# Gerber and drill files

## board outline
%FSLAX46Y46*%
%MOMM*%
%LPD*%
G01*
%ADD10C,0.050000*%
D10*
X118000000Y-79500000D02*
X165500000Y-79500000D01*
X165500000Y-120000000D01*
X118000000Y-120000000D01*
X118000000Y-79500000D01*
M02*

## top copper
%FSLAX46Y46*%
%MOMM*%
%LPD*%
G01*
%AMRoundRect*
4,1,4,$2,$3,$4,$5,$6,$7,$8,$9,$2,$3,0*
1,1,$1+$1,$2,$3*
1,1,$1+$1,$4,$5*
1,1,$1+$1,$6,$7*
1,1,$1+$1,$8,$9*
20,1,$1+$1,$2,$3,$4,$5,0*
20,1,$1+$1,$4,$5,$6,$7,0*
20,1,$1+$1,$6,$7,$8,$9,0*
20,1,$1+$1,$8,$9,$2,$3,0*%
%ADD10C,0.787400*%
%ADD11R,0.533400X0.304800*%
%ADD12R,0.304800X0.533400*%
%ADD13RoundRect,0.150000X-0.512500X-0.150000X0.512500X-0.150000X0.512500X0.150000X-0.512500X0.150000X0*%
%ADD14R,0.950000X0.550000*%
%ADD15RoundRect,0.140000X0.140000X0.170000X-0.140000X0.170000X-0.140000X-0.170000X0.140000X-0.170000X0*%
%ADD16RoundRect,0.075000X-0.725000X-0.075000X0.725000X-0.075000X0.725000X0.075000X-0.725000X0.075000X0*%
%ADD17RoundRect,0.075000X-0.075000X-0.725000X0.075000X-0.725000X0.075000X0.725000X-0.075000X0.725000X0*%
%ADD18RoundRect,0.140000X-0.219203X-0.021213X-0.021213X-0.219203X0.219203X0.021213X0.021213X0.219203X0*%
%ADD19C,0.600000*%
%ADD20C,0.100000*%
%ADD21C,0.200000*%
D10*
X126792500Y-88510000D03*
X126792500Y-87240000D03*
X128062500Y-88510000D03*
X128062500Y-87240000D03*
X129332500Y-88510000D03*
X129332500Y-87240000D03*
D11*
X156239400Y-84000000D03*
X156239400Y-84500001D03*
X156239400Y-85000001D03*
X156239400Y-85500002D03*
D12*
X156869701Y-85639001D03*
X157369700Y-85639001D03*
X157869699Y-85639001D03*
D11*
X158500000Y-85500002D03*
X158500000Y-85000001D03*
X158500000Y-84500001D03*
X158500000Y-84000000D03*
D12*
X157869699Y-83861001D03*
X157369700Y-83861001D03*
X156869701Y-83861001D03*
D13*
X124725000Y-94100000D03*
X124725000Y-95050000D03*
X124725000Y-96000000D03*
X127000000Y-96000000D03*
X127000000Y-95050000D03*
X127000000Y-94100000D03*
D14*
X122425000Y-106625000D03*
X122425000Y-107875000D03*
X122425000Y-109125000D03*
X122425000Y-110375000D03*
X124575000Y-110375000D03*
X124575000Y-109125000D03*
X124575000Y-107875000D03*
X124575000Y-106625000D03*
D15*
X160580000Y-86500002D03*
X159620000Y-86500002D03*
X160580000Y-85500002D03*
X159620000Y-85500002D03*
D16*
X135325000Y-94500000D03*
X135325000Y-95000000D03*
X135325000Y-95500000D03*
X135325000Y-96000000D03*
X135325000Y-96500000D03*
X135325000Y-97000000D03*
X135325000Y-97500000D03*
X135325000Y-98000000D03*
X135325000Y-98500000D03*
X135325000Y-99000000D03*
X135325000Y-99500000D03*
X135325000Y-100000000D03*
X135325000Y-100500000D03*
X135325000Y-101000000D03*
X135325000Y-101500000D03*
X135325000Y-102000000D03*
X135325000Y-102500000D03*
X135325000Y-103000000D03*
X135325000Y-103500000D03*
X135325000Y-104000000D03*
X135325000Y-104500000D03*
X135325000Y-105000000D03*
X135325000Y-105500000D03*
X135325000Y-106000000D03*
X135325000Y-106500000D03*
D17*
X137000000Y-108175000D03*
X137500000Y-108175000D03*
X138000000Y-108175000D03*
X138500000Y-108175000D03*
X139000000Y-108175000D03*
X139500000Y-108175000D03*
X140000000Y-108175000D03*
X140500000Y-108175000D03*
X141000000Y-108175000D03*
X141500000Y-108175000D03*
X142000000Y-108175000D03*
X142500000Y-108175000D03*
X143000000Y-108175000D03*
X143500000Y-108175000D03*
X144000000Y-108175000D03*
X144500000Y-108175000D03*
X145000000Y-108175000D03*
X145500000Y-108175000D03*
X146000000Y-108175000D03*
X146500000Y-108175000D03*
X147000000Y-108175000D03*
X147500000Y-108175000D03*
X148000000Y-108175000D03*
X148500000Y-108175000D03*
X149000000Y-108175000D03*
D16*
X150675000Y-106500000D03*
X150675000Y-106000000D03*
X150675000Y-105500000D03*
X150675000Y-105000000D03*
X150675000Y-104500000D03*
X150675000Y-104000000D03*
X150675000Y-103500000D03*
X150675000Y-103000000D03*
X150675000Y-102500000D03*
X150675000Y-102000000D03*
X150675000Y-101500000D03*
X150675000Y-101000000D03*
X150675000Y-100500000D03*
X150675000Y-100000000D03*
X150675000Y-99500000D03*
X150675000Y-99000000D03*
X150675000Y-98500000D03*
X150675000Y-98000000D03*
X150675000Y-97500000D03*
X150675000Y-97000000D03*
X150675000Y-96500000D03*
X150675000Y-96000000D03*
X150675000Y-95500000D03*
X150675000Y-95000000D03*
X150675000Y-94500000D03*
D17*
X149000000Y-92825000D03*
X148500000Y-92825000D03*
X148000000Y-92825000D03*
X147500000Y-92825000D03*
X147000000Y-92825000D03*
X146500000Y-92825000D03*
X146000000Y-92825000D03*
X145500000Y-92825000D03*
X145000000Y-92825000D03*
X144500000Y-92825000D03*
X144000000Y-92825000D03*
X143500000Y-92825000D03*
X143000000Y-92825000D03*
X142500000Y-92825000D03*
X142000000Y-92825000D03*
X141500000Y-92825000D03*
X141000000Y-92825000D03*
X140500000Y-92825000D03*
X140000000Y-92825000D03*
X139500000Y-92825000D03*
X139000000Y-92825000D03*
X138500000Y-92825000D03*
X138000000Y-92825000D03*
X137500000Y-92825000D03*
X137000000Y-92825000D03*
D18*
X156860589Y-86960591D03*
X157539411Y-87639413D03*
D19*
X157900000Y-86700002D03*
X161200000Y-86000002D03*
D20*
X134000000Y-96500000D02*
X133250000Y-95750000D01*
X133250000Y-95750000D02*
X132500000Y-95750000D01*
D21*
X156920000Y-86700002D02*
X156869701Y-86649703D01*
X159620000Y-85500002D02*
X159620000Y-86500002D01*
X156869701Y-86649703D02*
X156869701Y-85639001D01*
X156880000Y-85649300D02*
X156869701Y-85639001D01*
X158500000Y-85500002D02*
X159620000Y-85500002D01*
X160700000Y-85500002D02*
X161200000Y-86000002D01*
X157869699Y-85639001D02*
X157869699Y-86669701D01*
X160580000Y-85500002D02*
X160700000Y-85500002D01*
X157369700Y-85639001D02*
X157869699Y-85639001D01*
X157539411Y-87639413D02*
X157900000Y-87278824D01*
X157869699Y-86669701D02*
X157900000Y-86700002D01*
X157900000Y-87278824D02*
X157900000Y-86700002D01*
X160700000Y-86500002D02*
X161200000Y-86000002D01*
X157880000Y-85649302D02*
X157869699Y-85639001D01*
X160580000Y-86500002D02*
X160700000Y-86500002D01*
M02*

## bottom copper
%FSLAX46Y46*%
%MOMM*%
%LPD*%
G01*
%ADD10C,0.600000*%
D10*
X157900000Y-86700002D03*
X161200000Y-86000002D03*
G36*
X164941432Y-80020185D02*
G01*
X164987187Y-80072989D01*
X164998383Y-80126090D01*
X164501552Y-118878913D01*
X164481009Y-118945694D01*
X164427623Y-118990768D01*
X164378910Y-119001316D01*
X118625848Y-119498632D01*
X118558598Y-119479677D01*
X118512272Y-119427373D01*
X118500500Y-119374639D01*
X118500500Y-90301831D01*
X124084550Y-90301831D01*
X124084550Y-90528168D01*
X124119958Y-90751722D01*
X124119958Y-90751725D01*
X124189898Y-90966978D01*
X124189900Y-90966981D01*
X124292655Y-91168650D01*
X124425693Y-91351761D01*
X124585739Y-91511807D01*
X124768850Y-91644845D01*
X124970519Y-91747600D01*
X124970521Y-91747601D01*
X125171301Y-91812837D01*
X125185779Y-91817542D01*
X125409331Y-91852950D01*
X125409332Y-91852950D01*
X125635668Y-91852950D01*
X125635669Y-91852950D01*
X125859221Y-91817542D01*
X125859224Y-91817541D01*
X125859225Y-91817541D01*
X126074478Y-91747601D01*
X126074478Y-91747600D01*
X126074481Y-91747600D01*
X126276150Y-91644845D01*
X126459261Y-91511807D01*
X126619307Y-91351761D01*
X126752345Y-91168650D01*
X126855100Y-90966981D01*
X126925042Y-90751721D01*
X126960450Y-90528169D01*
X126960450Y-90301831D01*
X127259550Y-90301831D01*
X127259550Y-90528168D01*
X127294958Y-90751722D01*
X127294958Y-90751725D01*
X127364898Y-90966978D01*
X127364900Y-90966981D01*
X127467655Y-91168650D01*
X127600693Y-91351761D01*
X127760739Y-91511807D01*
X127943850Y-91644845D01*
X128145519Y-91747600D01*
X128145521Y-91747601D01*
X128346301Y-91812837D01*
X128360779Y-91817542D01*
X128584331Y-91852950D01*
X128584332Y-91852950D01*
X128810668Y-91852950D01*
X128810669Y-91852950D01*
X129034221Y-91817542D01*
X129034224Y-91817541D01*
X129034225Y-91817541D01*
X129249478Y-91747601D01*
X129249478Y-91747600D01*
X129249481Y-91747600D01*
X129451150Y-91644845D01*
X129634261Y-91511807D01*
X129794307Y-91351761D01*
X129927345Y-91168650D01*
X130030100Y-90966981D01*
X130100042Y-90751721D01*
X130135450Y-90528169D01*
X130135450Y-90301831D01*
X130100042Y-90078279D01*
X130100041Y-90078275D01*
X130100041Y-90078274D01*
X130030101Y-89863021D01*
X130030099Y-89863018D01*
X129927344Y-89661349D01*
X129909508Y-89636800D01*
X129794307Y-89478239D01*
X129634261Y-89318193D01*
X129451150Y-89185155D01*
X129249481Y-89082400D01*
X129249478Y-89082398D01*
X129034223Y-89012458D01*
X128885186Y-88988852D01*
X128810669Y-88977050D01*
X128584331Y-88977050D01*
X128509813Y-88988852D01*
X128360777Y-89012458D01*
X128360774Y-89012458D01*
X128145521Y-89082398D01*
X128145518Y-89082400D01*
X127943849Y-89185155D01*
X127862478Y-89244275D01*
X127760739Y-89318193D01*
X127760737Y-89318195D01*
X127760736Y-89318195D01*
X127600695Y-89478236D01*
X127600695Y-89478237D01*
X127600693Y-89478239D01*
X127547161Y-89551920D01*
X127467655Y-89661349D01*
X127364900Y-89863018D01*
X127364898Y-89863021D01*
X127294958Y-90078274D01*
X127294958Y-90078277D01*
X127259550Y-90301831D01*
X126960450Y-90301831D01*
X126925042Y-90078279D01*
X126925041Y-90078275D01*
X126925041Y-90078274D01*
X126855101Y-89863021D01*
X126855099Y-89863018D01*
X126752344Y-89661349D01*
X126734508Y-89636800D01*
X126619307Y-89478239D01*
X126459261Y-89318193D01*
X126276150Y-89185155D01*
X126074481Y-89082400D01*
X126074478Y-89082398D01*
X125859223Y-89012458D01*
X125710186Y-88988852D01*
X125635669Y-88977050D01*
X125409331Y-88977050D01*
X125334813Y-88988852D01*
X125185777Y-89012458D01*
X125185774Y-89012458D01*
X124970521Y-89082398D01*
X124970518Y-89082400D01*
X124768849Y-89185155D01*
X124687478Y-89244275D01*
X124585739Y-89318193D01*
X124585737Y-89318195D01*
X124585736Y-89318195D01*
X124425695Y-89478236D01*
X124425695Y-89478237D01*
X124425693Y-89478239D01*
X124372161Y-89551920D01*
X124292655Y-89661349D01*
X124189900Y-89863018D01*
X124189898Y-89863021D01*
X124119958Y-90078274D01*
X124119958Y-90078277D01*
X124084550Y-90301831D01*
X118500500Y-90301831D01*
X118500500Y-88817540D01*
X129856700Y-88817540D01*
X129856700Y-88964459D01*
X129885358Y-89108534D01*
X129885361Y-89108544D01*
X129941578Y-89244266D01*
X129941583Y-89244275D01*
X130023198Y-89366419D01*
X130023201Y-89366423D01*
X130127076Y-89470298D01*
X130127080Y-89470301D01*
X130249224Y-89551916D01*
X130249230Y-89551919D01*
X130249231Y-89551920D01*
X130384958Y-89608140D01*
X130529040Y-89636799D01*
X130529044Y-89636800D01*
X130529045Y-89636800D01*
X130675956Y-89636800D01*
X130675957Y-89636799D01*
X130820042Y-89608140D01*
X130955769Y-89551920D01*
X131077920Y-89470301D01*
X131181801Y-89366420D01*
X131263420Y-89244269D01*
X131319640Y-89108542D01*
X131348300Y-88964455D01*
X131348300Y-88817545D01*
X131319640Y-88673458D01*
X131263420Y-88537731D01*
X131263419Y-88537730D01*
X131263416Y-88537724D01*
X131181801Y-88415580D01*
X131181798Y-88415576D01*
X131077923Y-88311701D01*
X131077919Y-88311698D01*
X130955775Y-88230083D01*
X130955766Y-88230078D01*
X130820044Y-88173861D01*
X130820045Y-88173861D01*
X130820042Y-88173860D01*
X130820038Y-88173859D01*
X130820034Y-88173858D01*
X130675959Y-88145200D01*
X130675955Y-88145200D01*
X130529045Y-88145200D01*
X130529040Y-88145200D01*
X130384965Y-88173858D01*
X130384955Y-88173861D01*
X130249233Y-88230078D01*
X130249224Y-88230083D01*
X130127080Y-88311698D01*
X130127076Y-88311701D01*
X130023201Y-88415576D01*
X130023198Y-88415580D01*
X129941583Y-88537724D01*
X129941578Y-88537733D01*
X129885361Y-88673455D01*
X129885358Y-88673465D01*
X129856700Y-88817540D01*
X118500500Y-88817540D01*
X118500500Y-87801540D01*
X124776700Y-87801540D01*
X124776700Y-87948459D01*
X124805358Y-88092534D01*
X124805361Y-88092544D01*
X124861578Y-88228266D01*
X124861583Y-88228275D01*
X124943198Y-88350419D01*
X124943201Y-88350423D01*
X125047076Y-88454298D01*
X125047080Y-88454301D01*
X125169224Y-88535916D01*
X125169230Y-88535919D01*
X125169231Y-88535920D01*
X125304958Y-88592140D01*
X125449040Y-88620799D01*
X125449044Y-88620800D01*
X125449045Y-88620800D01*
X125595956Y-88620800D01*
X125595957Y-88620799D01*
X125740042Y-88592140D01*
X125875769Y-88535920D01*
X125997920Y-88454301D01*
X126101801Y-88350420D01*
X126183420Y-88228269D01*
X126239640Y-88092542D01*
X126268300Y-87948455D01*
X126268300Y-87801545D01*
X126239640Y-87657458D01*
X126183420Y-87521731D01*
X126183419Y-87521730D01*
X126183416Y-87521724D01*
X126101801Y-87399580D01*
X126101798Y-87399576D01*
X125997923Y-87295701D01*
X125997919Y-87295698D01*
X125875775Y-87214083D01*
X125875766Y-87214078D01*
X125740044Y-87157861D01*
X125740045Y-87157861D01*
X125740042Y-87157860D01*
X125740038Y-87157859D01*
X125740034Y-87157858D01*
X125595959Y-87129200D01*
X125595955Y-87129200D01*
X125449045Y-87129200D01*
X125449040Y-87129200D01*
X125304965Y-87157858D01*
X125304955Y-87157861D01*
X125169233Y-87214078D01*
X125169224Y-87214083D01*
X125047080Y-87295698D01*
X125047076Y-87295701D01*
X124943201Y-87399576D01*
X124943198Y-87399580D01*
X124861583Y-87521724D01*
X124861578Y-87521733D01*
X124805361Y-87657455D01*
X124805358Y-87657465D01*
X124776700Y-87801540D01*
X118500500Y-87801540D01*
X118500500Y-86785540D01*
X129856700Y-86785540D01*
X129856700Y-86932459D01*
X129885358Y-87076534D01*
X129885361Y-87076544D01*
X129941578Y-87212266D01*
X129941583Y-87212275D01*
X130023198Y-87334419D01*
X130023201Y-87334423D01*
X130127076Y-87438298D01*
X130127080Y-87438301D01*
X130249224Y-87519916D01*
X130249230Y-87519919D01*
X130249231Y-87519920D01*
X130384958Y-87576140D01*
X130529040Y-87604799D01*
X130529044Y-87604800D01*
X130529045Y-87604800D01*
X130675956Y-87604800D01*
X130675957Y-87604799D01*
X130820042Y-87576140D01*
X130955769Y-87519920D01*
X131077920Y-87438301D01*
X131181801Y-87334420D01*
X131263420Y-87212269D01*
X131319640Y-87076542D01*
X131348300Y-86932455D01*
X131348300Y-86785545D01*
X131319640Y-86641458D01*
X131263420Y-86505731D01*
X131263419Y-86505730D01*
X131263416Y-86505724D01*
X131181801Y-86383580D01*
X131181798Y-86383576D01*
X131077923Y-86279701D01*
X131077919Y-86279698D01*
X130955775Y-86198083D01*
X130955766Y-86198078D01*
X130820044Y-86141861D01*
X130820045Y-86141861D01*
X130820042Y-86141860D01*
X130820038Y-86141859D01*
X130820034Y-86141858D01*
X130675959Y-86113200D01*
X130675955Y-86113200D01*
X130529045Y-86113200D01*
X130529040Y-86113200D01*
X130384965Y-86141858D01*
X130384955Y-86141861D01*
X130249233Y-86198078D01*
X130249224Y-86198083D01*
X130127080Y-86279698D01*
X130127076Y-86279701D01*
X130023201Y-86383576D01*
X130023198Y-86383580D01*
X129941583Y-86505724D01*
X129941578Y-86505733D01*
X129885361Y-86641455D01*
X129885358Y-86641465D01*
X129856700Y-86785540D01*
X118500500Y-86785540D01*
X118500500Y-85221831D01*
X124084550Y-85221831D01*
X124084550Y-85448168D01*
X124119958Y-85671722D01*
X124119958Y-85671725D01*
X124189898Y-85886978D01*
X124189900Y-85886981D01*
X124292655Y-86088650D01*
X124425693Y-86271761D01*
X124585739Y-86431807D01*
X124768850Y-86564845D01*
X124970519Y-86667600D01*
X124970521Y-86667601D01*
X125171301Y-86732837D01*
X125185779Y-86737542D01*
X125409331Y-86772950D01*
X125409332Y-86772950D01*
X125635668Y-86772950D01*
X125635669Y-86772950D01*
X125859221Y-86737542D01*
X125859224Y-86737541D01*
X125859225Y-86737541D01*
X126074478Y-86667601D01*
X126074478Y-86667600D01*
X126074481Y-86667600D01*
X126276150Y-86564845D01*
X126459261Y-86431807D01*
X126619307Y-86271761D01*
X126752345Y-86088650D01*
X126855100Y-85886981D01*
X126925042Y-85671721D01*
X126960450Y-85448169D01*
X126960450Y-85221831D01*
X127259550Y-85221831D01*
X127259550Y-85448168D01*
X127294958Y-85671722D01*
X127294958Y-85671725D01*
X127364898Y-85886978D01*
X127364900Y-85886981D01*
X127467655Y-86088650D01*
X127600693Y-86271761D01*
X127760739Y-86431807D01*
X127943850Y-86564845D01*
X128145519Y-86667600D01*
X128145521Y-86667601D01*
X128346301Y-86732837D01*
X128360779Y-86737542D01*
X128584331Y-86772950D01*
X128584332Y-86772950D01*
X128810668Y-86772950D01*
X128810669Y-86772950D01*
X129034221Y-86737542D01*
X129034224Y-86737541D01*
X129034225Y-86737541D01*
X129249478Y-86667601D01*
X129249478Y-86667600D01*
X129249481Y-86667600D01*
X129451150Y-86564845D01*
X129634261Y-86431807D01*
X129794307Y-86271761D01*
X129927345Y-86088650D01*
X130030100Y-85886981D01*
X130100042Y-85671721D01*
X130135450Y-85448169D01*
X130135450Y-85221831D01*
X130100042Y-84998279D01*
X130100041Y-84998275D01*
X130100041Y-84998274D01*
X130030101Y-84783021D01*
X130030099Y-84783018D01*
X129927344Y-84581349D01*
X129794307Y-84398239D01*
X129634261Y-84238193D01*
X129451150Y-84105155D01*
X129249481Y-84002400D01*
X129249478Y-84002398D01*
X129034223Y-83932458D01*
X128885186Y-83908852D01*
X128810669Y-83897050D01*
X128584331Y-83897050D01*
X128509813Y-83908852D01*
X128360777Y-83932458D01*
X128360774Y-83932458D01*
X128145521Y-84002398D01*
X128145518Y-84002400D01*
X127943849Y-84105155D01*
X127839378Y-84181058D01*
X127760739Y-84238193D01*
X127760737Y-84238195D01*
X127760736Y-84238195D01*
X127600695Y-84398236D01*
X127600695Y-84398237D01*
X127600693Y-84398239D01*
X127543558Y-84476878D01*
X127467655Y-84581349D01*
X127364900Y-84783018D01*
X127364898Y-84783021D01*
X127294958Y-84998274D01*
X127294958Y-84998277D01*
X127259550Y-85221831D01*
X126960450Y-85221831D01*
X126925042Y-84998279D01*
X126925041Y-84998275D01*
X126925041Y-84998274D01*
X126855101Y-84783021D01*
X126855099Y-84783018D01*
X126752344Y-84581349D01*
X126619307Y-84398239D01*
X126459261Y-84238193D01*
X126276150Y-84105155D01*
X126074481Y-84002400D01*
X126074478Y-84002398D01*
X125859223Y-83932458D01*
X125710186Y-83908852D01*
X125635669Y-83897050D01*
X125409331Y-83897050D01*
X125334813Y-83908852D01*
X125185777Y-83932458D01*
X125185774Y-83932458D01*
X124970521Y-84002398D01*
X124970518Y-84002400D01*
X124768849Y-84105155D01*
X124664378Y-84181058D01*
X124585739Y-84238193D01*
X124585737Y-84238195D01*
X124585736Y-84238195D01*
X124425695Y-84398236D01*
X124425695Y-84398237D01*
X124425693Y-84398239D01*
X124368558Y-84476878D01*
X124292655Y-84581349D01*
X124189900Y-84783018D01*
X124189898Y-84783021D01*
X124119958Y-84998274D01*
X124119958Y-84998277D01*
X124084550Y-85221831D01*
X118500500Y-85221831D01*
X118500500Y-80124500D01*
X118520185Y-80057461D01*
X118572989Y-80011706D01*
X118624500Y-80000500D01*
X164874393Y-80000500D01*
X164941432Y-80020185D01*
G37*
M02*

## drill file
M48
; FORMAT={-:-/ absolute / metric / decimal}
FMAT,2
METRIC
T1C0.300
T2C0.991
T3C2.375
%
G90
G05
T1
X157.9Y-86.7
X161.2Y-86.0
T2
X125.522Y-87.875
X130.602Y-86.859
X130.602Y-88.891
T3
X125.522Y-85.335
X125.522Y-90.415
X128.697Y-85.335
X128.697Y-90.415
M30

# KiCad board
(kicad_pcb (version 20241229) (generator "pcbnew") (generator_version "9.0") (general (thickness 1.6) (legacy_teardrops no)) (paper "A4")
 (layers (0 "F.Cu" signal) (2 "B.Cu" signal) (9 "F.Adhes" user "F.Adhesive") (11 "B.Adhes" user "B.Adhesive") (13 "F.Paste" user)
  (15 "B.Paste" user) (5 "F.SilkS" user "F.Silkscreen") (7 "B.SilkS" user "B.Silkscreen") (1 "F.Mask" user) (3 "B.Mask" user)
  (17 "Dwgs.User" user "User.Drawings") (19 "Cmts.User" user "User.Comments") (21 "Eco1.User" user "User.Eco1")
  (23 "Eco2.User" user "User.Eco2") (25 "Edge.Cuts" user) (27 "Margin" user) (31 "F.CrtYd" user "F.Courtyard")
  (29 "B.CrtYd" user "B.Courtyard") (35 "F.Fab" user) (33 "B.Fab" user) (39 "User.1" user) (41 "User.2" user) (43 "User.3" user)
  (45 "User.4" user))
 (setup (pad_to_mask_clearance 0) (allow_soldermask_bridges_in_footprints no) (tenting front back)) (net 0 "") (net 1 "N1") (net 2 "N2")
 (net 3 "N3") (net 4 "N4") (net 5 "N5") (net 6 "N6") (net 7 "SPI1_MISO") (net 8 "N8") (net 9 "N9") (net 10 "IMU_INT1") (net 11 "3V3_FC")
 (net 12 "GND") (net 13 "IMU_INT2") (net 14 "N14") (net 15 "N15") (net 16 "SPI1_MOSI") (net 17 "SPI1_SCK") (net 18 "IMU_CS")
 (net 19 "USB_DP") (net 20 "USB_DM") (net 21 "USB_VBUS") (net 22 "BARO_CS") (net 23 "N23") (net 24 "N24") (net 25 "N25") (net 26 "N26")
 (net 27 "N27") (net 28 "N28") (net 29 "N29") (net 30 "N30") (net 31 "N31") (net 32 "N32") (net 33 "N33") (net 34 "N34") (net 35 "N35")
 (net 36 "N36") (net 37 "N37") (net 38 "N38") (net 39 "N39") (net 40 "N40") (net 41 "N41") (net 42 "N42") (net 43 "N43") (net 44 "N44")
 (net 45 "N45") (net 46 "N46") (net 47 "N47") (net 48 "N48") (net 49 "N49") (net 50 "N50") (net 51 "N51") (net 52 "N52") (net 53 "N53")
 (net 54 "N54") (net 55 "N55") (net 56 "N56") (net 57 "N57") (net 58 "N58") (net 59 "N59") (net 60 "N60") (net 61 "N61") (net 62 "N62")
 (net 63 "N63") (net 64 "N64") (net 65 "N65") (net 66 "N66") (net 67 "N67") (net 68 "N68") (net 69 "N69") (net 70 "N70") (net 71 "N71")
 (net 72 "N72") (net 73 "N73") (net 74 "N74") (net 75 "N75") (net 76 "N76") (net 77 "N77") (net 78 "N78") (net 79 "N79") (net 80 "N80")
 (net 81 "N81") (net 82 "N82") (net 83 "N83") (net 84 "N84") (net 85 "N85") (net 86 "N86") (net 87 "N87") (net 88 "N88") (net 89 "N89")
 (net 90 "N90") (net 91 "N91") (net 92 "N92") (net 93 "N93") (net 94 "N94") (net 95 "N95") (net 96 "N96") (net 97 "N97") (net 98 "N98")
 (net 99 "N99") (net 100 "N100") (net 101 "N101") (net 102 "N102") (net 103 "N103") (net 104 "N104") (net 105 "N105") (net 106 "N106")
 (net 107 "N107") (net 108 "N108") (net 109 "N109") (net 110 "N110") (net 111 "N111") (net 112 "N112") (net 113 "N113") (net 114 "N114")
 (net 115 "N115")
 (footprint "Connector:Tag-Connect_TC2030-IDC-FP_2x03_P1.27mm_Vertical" (layer "F.Cu") (at 128.0625 87.875)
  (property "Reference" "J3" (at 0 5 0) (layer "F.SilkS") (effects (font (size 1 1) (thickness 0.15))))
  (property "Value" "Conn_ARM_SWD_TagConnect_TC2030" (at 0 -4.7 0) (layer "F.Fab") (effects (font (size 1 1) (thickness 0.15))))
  (pad "" np_thru_hole circle (at -2.54 -2.54) (size 2.3749 2.3749) (drill 2.3749) (layers "*.Cu" "*.Mask"))
  (pad "" np_thru_hole circle (at -2.54 0) (size 0.9906 0.9906) (drill 0.9906) (layers "*.Cu" "*.Mask"))
  (pad "" np_thru_hole circle (at -2.54 2.54) (size 2.3749 2.3749) (drill 2.3749) (layers "*.Cu" "*.Mask"))
  (pad "" np_thru_hole circle (at 0.635 -2.54) (size 2.3749 2.3749) (drill 2.3749) (layers "*.Cu" "*.Mask"))
  (pad "" np_thru_hole circle (at 0.635 2.54) (size 2.3749 2.3749) (drill 2.3749) (layers "*.Cu" "*.Mask"))
  (pad "" np_thru_hole circle (at 2.54 -1.016) (size 0.9906 0.9906) (drill 0.9906) (layers "*.Cu" "*.Mask"))
  (pad "" np_thru_hole circle (at 2.54 1.016) (size 0.9906 0.9906) (drill 0.9906) (layers "*.Cu" "*.Mask"))
  (pad "1" connect circle (at -1.27 0.635) (size 0.7874 0.7874) (layers "F.Cu" "F.Mask") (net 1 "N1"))
  (pad "2" connect circle (at -1.27 -0.635) (size 0.7874 0.7874) (layers "F.Cu" "F.Mask") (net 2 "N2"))
  (pad "3" connect circle (at 0 0.635) (size 0.7874 0.7874) (layers "F.Cu" "F.Mask") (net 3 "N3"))
  (pad "4" connect circle (at 0 -0.635) (size 0.7874 0.7874) (layers "F.Cu" "F.Mask") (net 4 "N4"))
  (pad "5" connect circle (at 1.27 0.635) (size 0.7874 0.7874) (layers "F.Cu" "F.Mask") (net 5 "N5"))
  (pad "6" connect circle (at 1.27 -0.635) (size 0.7874 0.7874) (layers "F.Cu" "F.Mask") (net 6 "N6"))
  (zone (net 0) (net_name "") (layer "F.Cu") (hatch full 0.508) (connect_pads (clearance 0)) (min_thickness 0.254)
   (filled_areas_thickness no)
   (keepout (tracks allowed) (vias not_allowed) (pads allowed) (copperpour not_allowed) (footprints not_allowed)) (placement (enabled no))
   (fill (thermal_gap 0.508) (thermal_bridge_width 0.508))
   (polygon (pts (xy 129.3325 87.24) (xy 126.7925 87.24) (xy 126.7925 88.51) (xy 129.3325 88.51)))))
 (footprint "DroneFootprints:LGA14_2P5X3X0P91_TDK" (layer "F.Cu") (at 157.3697 84.750001)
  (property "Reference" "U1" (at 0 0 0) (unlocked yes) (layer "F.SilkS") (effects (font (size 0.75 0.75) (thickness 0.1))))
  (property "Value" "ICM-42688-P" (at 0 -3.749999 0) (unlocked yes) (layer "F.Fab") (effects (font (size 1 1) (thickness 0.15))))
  (pad "1" smd rect (at -1.1303 -0.750001 90) (size 0.3048 0.5334) (layers "F.Cu" "F.Mask" "F.Paste") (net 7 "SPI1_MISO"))
  (pad "2" smd rect (at -1.1303 -0.25 90) (size 0.3048 0.5334) (layers "F.Cu" "F.Mask" "F.Paste") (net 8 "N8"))
  (pad "3" smd rect (at -1.1303 0.25 90) (size 0.3048 0.5334) (layers "F.Cu" "F.Mask" "F.Paste") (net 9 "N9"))
  (pad "4" smd rect (at -1.1303 0.750001 90) (size 0.3048 0.5334) (layers "F.Cu" "F.Mask" "F.Paste") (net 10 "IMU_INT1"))
  (pad "5" smd rect (at -0.499999 0.889) (size 0.3048 0.5334) (layers "F.Cu" "F.Mask" "F.Paste") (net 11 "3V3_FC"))
  (pad "6" smd rect (at 0 0.889) (size 0.3048 0.5334) (layers "F.Cu" "F.Mask" "F.Paste") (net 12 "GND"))
  (pad "7" smd rect (at 0.499999 0.889) (size 0.3048 0.5334) (layers "F.Cu" "F.Mask" "F.Paste") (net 12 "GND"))
  (pad "8" smd rect (at 1.1303 0.750001 90) (size 0.3048 0.5334) (layers "F.Cu" "F.Mask" "F.Paste") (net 11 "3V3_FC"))
  (pad "9" smd rect (at 1.1303 0.25 90) (size 0.3048 0.5334) (layers "F.Cu" "F.Mask" "F.Paste") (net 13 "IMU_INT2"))
  (pad "10" smd rect (at 1.1303 -0.25 90) (size 0.3048 0.5334) (layers "F.Cu" "F.Mask" "F.Paste") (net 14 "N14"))
  (pad "11" smd rect (at 1.1303 -0.750001 90) (size 0.3048 0.5334) (layers "F.Cu" "F.Mask" "F.Paste") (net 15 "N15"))
  (pad "12" smd rect (at 0.499999 -0.889) (size 0.3048 0.5334) (layers "F.Cu" "F.Mask" "F.Paste") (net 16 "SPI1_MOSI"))
  (pad "13" smd rect (at 0 -0.889) (size 0.3048 0.5334) (layers "F.Cu" "F.Mask" "F.Paste") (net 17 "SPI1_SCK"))
  (pad "14" smd rect (at -0.499999 -0.889) (size 0.3048 0.5334) (layers "F.Cu" "F.Mask" "F.Paste") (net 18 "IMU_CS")))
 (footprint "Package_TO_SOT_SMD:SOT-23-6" (layer "F.Cu") (at 125.8625 95.05)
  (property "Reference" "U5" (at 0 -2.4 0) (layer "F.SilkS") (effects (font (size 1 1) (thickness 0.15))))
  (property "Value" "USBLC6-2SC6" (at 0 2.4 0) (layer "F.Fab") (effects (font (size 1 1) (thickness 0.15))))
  (pad "1" smd roundrect (at -1.1375 -0.95) (size 1.325 0.6) (layers "F.Cu" "F.Mask" "F.Paste") (roundrect_rratio 0.25) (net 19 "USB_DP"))
  (pad "2" smd roundrect (at -1.1375 0) (size 1.325 0.6) (layers "F.Cu" "F.Mask" "F.Paste") (roundrect_rratio 0.25) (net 12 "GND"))
  (pad "3" smd roundrect (at -1.1375 0.95) (size 1.325 0.6) (layers "F.Cu" "F.Mask" "F.Paste") (roundrect_rratio 0.25) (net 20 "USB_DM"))
  (pad "4" smd roundrect (at 1.1375 0.95) (size 1.325 0.6) (layers "F.Cu" "F.Mask" "F.Paste") (roundrect_rratio 0.25) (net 20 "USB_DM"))
  (pad "5" smd roundrect (at 1.1375 0) (size 1.325 0.6) (layers "F.Cu" "F.Mask" "F.Paste") (roundrect_rratio 0.25) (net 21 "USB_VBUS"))
  (pad "6" smd roundrect (at 1.1375 -0.95) (size 1.325 0.6) (layers "F.Cu" "F.Mask" "F.Paste") (roundrect_rratio 0.25) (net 19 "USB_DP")))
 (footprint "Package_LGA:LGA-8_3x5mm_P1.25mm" (layer "F.Cu") (at 123.5 108.5)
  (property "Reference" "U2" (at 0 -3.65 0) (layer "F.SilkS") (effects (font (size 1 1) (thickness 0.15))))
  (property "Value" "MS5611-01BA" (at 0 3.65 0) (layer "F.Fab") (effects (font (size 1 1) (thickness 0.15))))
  (pad "1" smd rect (at -1.075 -1.875) (size 0.95 0.55) (layers "F.Cu" "F.Mask" "F.Paste") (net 11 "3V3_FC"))
  (pad "2" smd rect (at -1.075 -0.625) (size 0.95 0.55) (layers "F.Cu" "F.Mask" "F.Paste") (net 12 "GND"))
  (pad "3" smd rect (at -1.075 0.625) (size 0.95 0.55) (layers "F.Cu" "F.Mask" "F.Paste") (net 12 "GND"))
  (pad "4" smd rect (at -1.075 1.875) (size 0.95 0.55) (layers "F.Cu" "F.Mask" "F.Paste") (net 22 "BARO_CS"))
  (pad "5" smd rect (at 1.075 1.875) (size 0.95 0.55) (layers "F.Cu" "F.Mask" "F.Paste") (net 22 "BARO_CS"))
  (pad "6" smd rect (at 1.075 0.625) (size 0.95 0.55) (layers "F.Cu" "F.Mask" "F.Paste") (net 17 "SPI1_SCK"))
  (pad "7" smd rect (at 1.075 -0.625) (size 0.95 0.55) (layers "F.Cu" "F.Mask" "F.Paste") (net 16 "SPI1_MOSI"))
  (pad "8" smd rect (at 1.075 -1.875) (size 0.95 0.55) (layers "F.Cu" "F.Mask" "F.Paste") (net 7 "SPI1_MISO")))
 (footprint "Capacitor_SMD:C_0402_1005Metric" (layer "F.Cu") (at 160.1 86.500002 180)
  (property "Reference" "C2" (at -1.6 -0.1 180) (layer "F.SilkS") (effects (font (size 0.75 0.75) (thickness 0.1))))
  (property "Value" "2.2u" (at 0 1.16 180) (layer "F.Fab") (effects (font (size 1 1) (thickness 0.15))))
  (pad "1" smd roundrect (at -0.48 0 180) (size 0.56 0.62) (layers "F.Cu" "F.Mask" "F.Paste") (roundrect_rratio 0.25) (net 12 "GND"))
  (pad "2" smd roundrect (at 0.48 0 180) (size 0.56 0.62) (layers "F.Cu" "F.Mask" "F.Paste") (roundrect_rratio 0.25) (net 11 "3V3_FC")))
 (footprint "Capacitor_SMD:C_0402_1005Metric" (layer "F.Cu") (at 160.1 85.500002 180)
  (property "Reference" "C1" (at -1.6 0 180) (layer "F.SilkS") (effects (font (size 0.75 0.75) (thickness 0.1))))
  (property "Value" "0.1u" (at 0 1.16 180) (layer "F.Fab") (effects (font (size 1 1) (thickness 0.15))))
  (pad "1" smd roundrect (at -0.48 0 180) (size 0.56 0.62) (layers "F.Cu" "F.Mask" "F.Paste") (roundrect_rratio 0.25) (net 12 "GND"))
  (pad "2" smd roundrect (at 0.48 0 180) (size 0.56 0.62) (layers "F.Cu" "F.Mask" "F.Paste") (roundrect_rratio 0.25) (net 11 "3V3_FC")))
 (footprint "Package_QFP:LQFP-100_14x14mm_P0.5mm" (layer "F.Cu") (at 143 100.5)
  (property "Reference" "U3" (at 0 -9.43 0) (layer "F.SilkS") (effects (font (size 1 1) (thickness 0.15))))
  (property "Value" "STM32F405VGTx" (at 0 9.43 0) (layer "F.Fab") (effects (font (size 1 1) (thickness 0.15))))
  (pad "1" smd roundrect (at -7.675 -6) (size 1.6 0.3) (layers "F.Cu" "F.Mask" "F.Paste") (roundrect_rratio 0.25) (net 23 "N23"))
  (pad "2" smd roundrect (at -7.675 -5.5) (size 1.6 0.3) (layers "F.Cu" "F.Mask" "F.Paste") (roundrect_rratio 0.25) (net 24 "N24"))
  (pad "3" smd roundrect (at -7.675 -5) (size 1.6 0.3) (layers "F.Cu" "F.Mask" "F.Paste") (roundrect_rratio 0.25) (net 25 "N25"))
  (pad "4" smd roundrect (at -7.675 -4.5) (size 1.6 0.3) (layers "F.Cu" "F.Mask" "F.Paste") (roundrect_rratio 0.25) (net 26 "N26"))
  (pad "5" smd roundrect (at -7.675 -4) (size 1.6 0.3) (layers "F.Cu" "F.Mask" "F.Paste") (roundrect_rratio 0.25) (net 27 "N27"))
  (pad "6" smd roundrect (at -7.675 -3.5) (size 1.6 0.3) (layers "F.Cu" "F.Mask" "F.Paste") (roundrect_rratio 0.25) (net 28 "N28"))
  (pad "7" smd roundrect (at -7.675 -3) (size 1.6 0.3) (layers "F.Cu" "F.Mask" "F.Paste") (roundrect_rratio 0.25) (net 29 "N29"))
  (pad "8" smd roundrect (at -7.675 -2.5) (size 1.6 0.3) (layers "F.Cu" "F.Mask" "F.Paste") (roundrect_rratio 0.25) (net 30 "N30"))
  (pad "9" smd roundrect (at -7.675 -2) (size 1.6 0.3) (layers "F.Cu" "F.Mask" "F.Paste") (roundrect_rratio 0.25) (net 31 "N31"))
  (pad "10" smd roundrect (at -7.675 -1.5) (size 1.6 0.3) (layers "F.Cu" "F.Mask" "F.Paste") (roundrect_rratio 0.25) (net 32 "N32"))
  (pad "11" smd roundrect (at -7.675 -1) (size 1.6 0.3) (layers "F.Cu" "F.Mask" "F.Paste") (roundrect_rratio 0.25) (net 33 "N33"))
  (pad "12" smd roundrect (at -7.675 -0.5) (size 1.6 0.3) (layers "F.Cu" "F.Mask" "F.Paste") (roundrect_rratio 0.25) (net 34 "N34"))
  (pad "13" smd roundrect (at -7.675 0) (size 1.6 0.3) (layers "F.Cu" "F.Mask" "F.Paste") (roundrect_rratio 0.25) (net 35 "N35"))
  (pad "14" smd roundrect (at -7.675 0.5) (size 1.6 0.3) (layers "F.Cu" "F.Mask" "F.Paste") (roundrect_rratio 0.25) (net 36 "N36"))
  (pad "15" smd roundrect (at -7.675 1) (size 1.6 0.3) (layers "F.Cu" "F.Mask" "F.Paste") (roundrect_rratio 0.25) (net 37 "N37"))
  (pad "16" smd roundrect (at -7.675 1.5) (size 1.6 0.3) (layers "F.Cu" "F.Mask" "F.Paste") (roundrect_rratio 0.25) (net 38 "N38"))
  (pad "17" smd roundrect (at -7.675 2) (size 1.6 0.3) (layers "F.Cu" "F.Mask" "F.Paste") (roundrect_rratio 0.25) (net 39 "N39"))
  (pad "18" smd roundrect (at -7.675 2.5) (size 1.6 0.3) (layers "F.Cu" "F.Mask" "F.Paste") (roundrect_rratio 0.25) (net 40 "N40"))
  (pad "19" smd roundrect (at -7.675 3) (size 1.6 0.3) (layers "F.Cu" "F.Mask" "F.Paste") (roundrect_rratio 0.25) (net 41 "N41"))
  (pad "20" smd roundrect (at -7.675 3.5) (size 1.6 0.3) (layers "F.Cu" "F.Mask" "F.Paste") (roundrect_rratio 0.25) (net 12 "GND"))
  (pad "21" smd roundrect (at -7.675 4) (size 1.6 0.3) (layers "F.Cu" "F.Mask" "F.Paste") (roundrect_rratio 0.25) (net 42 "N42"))
  (pad "22" smd roundrect (at -7.675 4.5) (size 1.6 0.3) (layers "F.Cu" "F.Mask" "F.Paste") (roundrect_rratio 0.25) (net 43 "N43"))
  (pad "23" smd roundrect (at -7.675 5) (size 1.6 0.3) (layers "F.Cu" "F.Mask" "F.Paste") (roundrect_rratio 0.25) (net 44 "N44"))
  (pad "24" smd roundrect (at -7.675 5.5) (size 1.6 0.3) (layers "F.Cu" "F.Mask" "F.Paste") (roundrect_rratio 0.25) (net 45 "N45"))
  (pad "25" smd roundrect (at -7.675 6) (size 1.6 0.3) (layers "F.Cu" "F.Mask" "F.Paste") (roundrect_rratio 0.25) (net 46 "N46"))
  (pad "26" smd roundrect (at -6 7.675) (size 0.3 1.6) (layers "F.Cu" "F.Mask" "F.Paste") (roundrect_rratio 0.25) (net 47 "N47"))
  (pad "27" smd roundrect (at -5.5 7.675) (size 0.3 1.6) (layers "F.Cu" "F.Mask" "F.Paste") (roundrect_rratio 0.25) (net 32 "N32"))
  (pad "28" smd roundrect (at -5 7.675) (size 0.3 1.6) (layers "F.Cu" "F.Mask" "F.Paste") (roundrect_rratio 0.25) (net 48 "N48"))
  (pad "29" smd roundrect (at -4.5 7.675) (size 0.3 1.6) (layers "F.Cu" "F.Mask" "F.Paste") (roundrect_rratio 0.25) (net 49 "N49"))
  (pad "30" smd roundrect (at -4 7.675) (size 0.3 1.6) (layers "F.Cu" "F.Mask" "F.Paste") (roundrect_rratio 0.25) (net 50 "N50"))
  (pad "31" smd roundrect (at -3.5 7.675) (size 0.3 1.6) (layers "F.Cu" "F.Mask" "F.Paste") (roundrect_rratio 0.25) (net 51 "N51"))
  (pad "32" smd roundrect (at -3 7.675) (size 0.3 1.6) (layers "F.Cu" "F.Mask" "F.Paste") (roundrect_rratio 0.25) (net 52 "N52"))
  (pad "33" smd roundrect (at -2.5 7.675) (size 0.3 1.6) (layers "F.Cu" "F.Mask" "F.Paste") (roundrect_rratio 0.25) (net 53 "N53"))
  (pad "34" smd roundrect (at -2 7.675) (size 0.3 1.6) (layers "F.Cu" "F.Mask" "F.Paste") (roundrect_rratio 0.25) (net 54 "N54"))
  (pad "35" smd roundrect (at -1.5 7.675) (size 0.3 1.6) (layers "F.Cu" "F.Mask" "F.Paste") (roundrect_rratio 0.25) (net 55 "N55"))
  (pad "36" smd roundrect (at -1 7.675) (size 0.3 1.6) (layers "F.Cu" "F.Mask" "F.Paste") (roundrect_rratio 0.25) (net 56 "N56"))
  (pad "37" smd roundrect (at -0.5 7.675) (size 0.3 1.6) (layers "F.Cu" "F.Mask" "F.Paste") (roundrect_rratio 0.25) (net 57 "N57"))
  (pad "38" smd roundrect (at 0 7.675) (size 0.3 1.6) (layers "F.Cu" "F.Mask" "F.Paste") (roundrect_rratio 0.25) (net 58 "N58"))
  (pad "39" smd roundrect (at 0.5 7.675) (size 0.3 1.6) (layers "F.Cu" "F.Mask" "F.Paste") (roundrect_rratio 0.25) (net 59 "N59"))
  (pad "40" smd roundrect (at 1 7.675) (size 0.3 1.6) (layers "F.Cu" "F.Mask" "F.Paste") (roundrect_rratio 0.25) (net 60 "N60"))
  (pad "41" smd roundrect (at 1.5 7.675) (size 0.3 1.6) (layers "F.Cu" "F.Mask" "F.Paste") (roundrect_rratio 0.25) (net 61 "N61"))
  (pad "42" smd roundrect (at 2 7.675) (size 0.3 1.6) (layers "F.Cu" "F.Mask" "F.Paste") (roundrect_rratio 0.25) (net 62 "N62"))
  (pad "43" smd roundrect (at 2.5 7.675) (size 0.3 1.6) (layers "F.Cu" "F.Mask" "F.Paste") (roundrect_rratio 0.25) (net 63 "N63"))
  (pad "44" smd roundrect (at 3 7.675) (size 0.3 1.6) (layers "F.Cu" "F.Mask" "F.Paste") (roundrect_rratio 0.25) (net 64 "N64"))
  (pad "45" smd roundrect (at 3.5 7.675) (size 0.3 1.6) (layers "F.Cu" "F.Mask" "F.Paste") (roundrect_rratio 0.25) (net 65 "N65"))
  (pad "46" smd roundrect (at 4 7.675) (size 0.3 1.6) (layers "F.Cu" "F.Mask" "F.Paste") (roundrect_rratio 0.25) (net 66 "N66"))
  (pad "47" smd roundrect (at 4.5 7.675) (size 0.3 1.6) (layers "F.Cu" "F.Mask" "F.Paste") (roundrect_rratio 0.25) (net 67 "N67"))
  (pad "48" smd roundrect (at 5 7.675) (size 0.3 1.6) (layers "F.Cu" "F.Mask" "F.Paste") (roundrect_rratio 0.25) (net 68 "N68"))
  (pad "49" smd roundrect (at 5.5 7.675) (size 0.3 1.6) (layers "F.Cu" "F.Mask" "F.Paste") (roundrect_rratio 0.25) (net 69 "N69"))
  (pad "50" smd roundrect (at 6 7.675) (size 0.3 1.6) (layers "F.Cu" "F.Mask" "F.Paste") (roundrect_rratio 0.25) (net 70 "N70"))
  (pad "51" smd roundrect (at 7.675 6) (size 1.6 0.3) (layers "F.Cu" "F.Mask" "F.Paste") (roundrect_rratio 0.25) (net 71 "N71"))
  (pad "52" smd roundrect (at 7.675 5.5) (size 1.6 0.3) (layers "F.Cu" "F.Mask" "F.Paste") (roundrect_rratio 0.25) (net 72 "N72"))
  (pad "53" smd roundrect (at 7.675 5) (size 1.6 0.3) (layers "F.Cu" "F.Mask" "F.Paste") (roundrect_rratio 0.25) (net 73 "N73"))
  (pad "54" smd roundrect (at 7.675 4.5) (size 1.6 0.3) (layers "F.Cu" "F.Mask" "F.Paste") (roundrect_rratio 0.25) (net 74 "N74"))
  (pad "55" smd roundrect (at 7.675 4) (size 1.6 0.3) (layers "F.Cu" "F.Mask" "F.Paste") (roundrect_rratio 0.25) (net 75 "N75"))
  (pad "56" smd roundrect (at 7.675 3.5) (size 1.6 0.3) (layers "F.Cu" "F.Mask" "F.Paste") (roundrect_rratio 0.25) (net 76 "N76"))
  (pad "57" smd roundrect (at 7.675 3) (size 1.6 0.3) (layers "F.Cu" "F.Mask" "F.Paste") (roundrect_rratio 0.25) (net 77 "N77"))
  (pad "58" smd roundrect (at 7.675 2.5) (size 1.6 0.3) (layers "F.Cu" "F.Mask" "F.Paste") (roundrect_rratio 0.25) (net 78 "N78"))
  (pad "59" smd roundrect (at 7.675 2) (size 1.6 0.3) (layers "F.Cu" "F.Mask" "F.Paste") (roundrect_rratio 0.25) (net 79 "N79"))
  (pad "60" smd roundrect (at 7.675 1.5) (size 1.6 0.3) (layers "F.Cu" "F.Mask" "F.Paste") (roundrect_rratio 0.25) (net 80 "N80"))
  (pad "61" smd roundrect (at 7.675 1) (size 1.6 0.3) (layers "F.Cu" "F.Mask" "F.Paste") (roundrect_rratio 0.25) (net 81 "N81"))
  (pad "62" smd roundrect (at 7.675 0.5) (size 1.6 0.3) (layers "F.Cu" "F.Mask" "F.Paste") (roundrect_rratio 0.25) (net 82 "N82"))
  (pad "63" smd roundrect (at 7.675 0) (size 1.6 0.3) (layers "F.Cu" "F.Mask" "F.Paste") (roundrect_rratio 0.25) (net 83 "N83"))
  (pad "64" smd roundrect (at 7.675 -0.5) (size 1.6 0.3) (layers "F.Cu" "F.Mask" "F.Paste") (roundrect_rratio 0.25) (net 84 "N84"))
  (pad "65" smd roundrect (at 7.675 -1) (size 1.6 0.3) (layers "F.Cu" "F.Mask" "F.Paste") (roundrect_rratio 0.25) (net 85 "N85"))
  (pad "66" smd roundrect (at 7.675 -1.5) (size 1.6 0.3) (layers "F.Cu" "F.Mask" "F.Paste") (roundrect_rratio 0.25) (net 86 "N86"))
  (pad "67" smd roundrect (at 7.675 -2) (size 1.6 0.3) (layers "F.Cu" "F.Mask" "F.Paste") (roundrect_rratio 0.25) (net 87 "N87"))
  (pad "68" smd roundrect (at 7.675 -2.5) (size 1.6 0.3) (layers "F.Cu" "F.Mask" "F.Paste") (roundrect_rratio 0.25) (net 21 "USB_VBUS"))
  (pad "69" smd roundrect (at 7.675 -3) (size 1.6 0.3) (layers "F.Cu" "F.Mask" "F.Paste") (roundrect_rratio 0.25) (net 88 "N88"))
  (pad "70" smd roundrect (at 7.675 -3.5) (size 1.6 0.3) (layers "F.Cu" "F.Mask" "F.Paste") (roundrect_rratio 0.25) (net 20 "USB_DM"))
  (pad "71" smd roundrect (at 7.675 -4) (size 1.6 0.3) (layers "F.Cu" "F.Mask" "F.Paste") (roundrect_rratio 0.25) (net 19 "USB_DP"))
  (pad "72" smd roundrect (at 7.675 -4.5) (size 1.6 0.3) (layers "F.Cu" "F.Mask" "F.Paste") (roundrect_rratio 0.25) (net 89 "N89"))
  (pad "73" smd roundrect (at 7.675 -5) (size 1.6 0.3) (layers "F.Cu" "F.Mask" "F.Paste") (roundrect_rratio 0.25) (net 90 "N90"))
  (pad "74" smd roundrect (at 7.675 -5.5) (size 1.6 0.3) (layers "F.Cu" "F.Mask" "F.Paste") (roundrect_rratio 0.25) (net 32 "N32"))
  (pad "75" smd roundrect (at 7.675 -6) (size 1.6 0.3) (layers "F.Cu" "F.Mask" "F.Paste") (roundrect_rratio 0.25) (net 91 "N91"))
  (pad "76" smd roundrect (at 6 -7.675) (size 0.3 1.6) (layers "F.Cu" "F.Mask" "F.Paste") (roundrect_rratio 0.25) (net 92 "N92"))
  (pad "77" smd roundrect (at 5.5 -7.675) (size 0.3 1.6) (layers "F.Cu" "F.Mask" "F.Paste") (roundrect_rratio 0.25) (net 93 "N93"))
  (pad "78" smd roundrect (at 5 -7.675) (size 0.3 1.6) (layers "F.Cu" "F.Mask" "F.Paste") (roundrect_rratio 0.25) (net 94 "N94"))
  (pad "79" smd roundrect (at 4.5 -7.675) (size 0.3 1.6) (layers "F.Cu" "F.Mask" "F.Paste") (roundrect_rratio 0.25) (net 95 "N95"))
  (pad "80" smd roundrect (at 4 -7.675) (size 0.3 1.6) (layers "F.Cu" "F.Mask" "F.Paste") (roundrect_rratio 0.25) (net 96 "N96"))
  (pad "81" smd roundrect (at 3.5 -7.675) (size 0.3 1.6) (layers "F.Cu" "F.Mask" "F.Paste") (roundrect_rratio 0.25) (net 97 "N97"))
  (pad "82" smd roundrect (at 3 -7.675) (size 0.3 1.6) (layers "F.Cu" "F.Mask" "F.Paste") (roundrect_rratio 0.25) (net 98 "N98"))
  (pad "83" smd roundrect (at 2.5 -7.675) (size 0.3 1.6) (layers "F.Cu" "F.Mask" "F.Paste") (roundrect_rratio 0.25) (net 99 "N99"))
  (pad "84" smd roundrect (at 2 -7.675) (size 0.3 1.6) (layers "F.Cu" "F.Mask" "F.Paste") (roundrect_rratio 0.25) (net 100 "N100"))
  (pad "85" smd roundrect (at 1.5 -7.675) (size 0.3 1.6) (layers "F.Cu" "F.Mask" "F.Paste") (roundrect_rratio 0.25) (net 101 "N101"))
  (pad "86" smd roundrect (at 1 -7.675) (size 0.3 1.6) (layers "F.Cu" "F.Mask" "F.Paste") (roundrect_rratio 0.25) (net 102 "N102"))
  (pad "87" smd roundrect (at 0.5 -7.675) (size 0.3 1.6) (layers "F.Cu" "F.Mask" "F.Paste") (roundrect_rratio 0.25) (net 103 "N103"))
  (pad "88" smd roundrect (at 0 -7.675) (size 0.3 1.6) (layers "F.Cu" "F.Mask" "F.Paste") (roundrect_rratio 0.25) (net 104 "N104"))
  (pad "89" smd roundrect (at -0.5 -7.675) (size 0.3 1.6) (layers "F.Cu" "F.Mask" "F.Paste") (roundrect_rratio 0.25) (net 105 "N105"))
  (pad "90" smd roundrect (at -1 -7.675) (size 0.3 1.6) (layers "F.Cu" "F.Mask" "F.Paste") (roundrect_rratio 0.25) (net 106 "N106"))
  (pad "91" smd roundrect (at -1.5 -7.675) (size 0.3 1.6) (layers "F.Cu" "F.Mask" "F.Paste") (roundrect_rratio 0.25) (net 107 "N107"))
  (pad "92" smd roundrect (at -2 -7.675) (size 0.3 1.6) (layers "F.Cu" "F.Mask" "F.Paste") (roundrect_rratio 0.25) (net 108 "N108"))
  (pad "93" smd roundrect (at -2.5 -7.675) (size 0.3 1.6) (layers "F.Cu" "F.Mask" "F.Paste") (roundrect_rratio 0.25) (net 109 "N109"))
  (pad "94" smd roundrect (at -3 -7.675) (size 0.3 1.6) (layers "F.Cu" "F.Mask" "F.Paste") (roundrect_rratio 0.25) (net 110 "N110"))
  (pad "95" smd roundrect (at -3.5 -7.675) (size 0.3 1.6) (layers "F.Cu" "F.Mask" "F.Paste") (roundrect_rratio 0.25) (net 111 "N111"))
  (pad "96" smd roundrect (at -4 -7.675) (size 0.3 1.6) (layers "F.Cu" "F.Mask" "F.Paste") (roundrect_rratio 0.25) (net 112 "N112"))
  (pad "97" smd roundrect (at -4.5 -7.675) (size 0.3 1.6) (layers "F.Cu" "F.Mask" "F.Paste") (roundrect_rratio 0.25) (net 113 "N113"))
  (pad "98" smd roundrect (at -5 -7.675) (size 0.3 1.6) (layers "F.Cu" "F.Mask" "F.Paste") (roundrect_rratio 0.25) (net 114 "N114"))
  (pad "99" smd roundrect (at -5.5 -7.675) (size 0.3 1.6) (layers "F.Cu" "F.Mask" "F.Paste") (roundrect_rratio 0.25) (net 32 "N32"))
  (pad "100" smd roundrect (at -6 -7.675) (size 0.3 1.6) (layers "F.Cu" "F.Mask" "F.Paste") (roundrect_rratio 0.25) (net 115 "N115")))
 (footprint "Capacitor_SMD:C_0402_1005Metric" (layer "F.Cu") (at 157.2 87.300002 -45)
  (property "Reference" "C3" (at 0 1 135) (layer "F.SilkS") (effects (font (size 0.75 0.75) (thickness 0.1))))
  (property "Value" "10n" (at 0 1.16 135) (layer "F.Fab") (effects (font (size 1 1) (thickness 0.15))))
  (pad "1" smd roundrect (at -0.48 0 315) (size 0.56 0.62) (layers "F.Cu" "F.Mask" "F.Paste") (roundrect_rratio 0.25) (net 11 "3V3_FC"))
  (pad "2" smd roundrect (at 0.48 0 315) (size 0.56 0.62) (layers "F.Cu" "F.Mask" "F.Paste") (roundrect_rratio 0.25) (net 12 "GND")))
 (gr_rect (start 118 79.5) (end 165.5 120) (stroke (width 0.05) (type default)) (fill no) (layer "Edge.Cuts"))
 (segment (start 134 96.5) (end 133.25 95.75) (width 0.1) (layer "F.Cu") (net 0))
 (segment (start 133.25 95.75) (end 132.5 95.75) (width 0.1) (layer "F.Cu") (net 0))
 (segment (start 156.92 86.700002) (end 156.869701 86.649703) (width 0.2) (layer "F.Cu") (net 11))
 (segment (start 159.62 85.500002) (end 159.62 86.500002) (width 0.2) (layer "F.Cu") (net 11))
 (segment (start 156.869701 86.649703) (end 156.869701 85.639001) (width 0.2) (layer "F.Cu") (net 11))
 (segment (start 156.88 85.6493) (end 156.869701 85.639001) (width 0.2) (layer "F.Cu") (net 11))
 (segment (start 158.5 85.500002) (end 159.62 85.500002) (width 0.2) (layer "F.Cu") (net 11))
 (segment (start 160.7 85.500002) (end 161.2 86.000002) (width 0.2) (layer "F.Cu") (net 12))
 (segment (start 157.869699 85.639001) (end 157.869699 86.669701) (width 0.2) (layer "F.Cu") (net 12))
 (segment (start 160.58 85.500002) (end 160.7 85.500002) (width 0.2) (layer "F.Cu") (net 12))
 (segment (start 157.3697 85.639001) (end 157.869699 85.639001) (width 0.2) (layer "F.Cu") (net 12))
 (segment (start 157.539411 87.639413) (end 157.9 87.278824) (width 0.2) (layer "F.Cu") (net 12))
 (segment (start 157.869699 86.669701) (end 157.9 86.700002) (width 0.2) (layer "F.Cu") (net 12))
 (segment (start 157.9 87.278824) (end 157.9 86.700002) (width 0.2) (layer "F.Cu") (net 12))
 (segment (start 160.7 86.500002) (end 161.2 86.000002) (width 0.2) (layer "F.Cu") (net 12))
 (segment (start 157.88 85.649302) (end 157.869699 85.639001) (width 0.2) (layer "F.Cu") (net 12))
 (segment (start 160.58 86.500002) (end 160.7 86.500002) (width 0.2) (layer "F.Cu") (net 12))
 (via (at 157.9 86.700002) (size 0.6) (drill 0.3) (layers "F.Cu" "B.Cu") (free yes) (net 12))
 (via (at 161.2 86.000002) (size 0.6) (drill 0.3) (layers "F.Cu" "B.Cu") (free yes) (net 12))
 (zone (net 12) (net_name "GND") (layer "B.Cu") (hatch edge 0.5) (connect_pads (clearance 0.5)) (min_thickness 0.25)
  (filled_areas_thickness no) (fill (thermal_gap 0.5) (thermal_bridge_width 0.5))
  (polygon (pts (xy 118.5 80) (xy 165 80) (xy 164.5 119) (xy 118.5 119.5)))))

